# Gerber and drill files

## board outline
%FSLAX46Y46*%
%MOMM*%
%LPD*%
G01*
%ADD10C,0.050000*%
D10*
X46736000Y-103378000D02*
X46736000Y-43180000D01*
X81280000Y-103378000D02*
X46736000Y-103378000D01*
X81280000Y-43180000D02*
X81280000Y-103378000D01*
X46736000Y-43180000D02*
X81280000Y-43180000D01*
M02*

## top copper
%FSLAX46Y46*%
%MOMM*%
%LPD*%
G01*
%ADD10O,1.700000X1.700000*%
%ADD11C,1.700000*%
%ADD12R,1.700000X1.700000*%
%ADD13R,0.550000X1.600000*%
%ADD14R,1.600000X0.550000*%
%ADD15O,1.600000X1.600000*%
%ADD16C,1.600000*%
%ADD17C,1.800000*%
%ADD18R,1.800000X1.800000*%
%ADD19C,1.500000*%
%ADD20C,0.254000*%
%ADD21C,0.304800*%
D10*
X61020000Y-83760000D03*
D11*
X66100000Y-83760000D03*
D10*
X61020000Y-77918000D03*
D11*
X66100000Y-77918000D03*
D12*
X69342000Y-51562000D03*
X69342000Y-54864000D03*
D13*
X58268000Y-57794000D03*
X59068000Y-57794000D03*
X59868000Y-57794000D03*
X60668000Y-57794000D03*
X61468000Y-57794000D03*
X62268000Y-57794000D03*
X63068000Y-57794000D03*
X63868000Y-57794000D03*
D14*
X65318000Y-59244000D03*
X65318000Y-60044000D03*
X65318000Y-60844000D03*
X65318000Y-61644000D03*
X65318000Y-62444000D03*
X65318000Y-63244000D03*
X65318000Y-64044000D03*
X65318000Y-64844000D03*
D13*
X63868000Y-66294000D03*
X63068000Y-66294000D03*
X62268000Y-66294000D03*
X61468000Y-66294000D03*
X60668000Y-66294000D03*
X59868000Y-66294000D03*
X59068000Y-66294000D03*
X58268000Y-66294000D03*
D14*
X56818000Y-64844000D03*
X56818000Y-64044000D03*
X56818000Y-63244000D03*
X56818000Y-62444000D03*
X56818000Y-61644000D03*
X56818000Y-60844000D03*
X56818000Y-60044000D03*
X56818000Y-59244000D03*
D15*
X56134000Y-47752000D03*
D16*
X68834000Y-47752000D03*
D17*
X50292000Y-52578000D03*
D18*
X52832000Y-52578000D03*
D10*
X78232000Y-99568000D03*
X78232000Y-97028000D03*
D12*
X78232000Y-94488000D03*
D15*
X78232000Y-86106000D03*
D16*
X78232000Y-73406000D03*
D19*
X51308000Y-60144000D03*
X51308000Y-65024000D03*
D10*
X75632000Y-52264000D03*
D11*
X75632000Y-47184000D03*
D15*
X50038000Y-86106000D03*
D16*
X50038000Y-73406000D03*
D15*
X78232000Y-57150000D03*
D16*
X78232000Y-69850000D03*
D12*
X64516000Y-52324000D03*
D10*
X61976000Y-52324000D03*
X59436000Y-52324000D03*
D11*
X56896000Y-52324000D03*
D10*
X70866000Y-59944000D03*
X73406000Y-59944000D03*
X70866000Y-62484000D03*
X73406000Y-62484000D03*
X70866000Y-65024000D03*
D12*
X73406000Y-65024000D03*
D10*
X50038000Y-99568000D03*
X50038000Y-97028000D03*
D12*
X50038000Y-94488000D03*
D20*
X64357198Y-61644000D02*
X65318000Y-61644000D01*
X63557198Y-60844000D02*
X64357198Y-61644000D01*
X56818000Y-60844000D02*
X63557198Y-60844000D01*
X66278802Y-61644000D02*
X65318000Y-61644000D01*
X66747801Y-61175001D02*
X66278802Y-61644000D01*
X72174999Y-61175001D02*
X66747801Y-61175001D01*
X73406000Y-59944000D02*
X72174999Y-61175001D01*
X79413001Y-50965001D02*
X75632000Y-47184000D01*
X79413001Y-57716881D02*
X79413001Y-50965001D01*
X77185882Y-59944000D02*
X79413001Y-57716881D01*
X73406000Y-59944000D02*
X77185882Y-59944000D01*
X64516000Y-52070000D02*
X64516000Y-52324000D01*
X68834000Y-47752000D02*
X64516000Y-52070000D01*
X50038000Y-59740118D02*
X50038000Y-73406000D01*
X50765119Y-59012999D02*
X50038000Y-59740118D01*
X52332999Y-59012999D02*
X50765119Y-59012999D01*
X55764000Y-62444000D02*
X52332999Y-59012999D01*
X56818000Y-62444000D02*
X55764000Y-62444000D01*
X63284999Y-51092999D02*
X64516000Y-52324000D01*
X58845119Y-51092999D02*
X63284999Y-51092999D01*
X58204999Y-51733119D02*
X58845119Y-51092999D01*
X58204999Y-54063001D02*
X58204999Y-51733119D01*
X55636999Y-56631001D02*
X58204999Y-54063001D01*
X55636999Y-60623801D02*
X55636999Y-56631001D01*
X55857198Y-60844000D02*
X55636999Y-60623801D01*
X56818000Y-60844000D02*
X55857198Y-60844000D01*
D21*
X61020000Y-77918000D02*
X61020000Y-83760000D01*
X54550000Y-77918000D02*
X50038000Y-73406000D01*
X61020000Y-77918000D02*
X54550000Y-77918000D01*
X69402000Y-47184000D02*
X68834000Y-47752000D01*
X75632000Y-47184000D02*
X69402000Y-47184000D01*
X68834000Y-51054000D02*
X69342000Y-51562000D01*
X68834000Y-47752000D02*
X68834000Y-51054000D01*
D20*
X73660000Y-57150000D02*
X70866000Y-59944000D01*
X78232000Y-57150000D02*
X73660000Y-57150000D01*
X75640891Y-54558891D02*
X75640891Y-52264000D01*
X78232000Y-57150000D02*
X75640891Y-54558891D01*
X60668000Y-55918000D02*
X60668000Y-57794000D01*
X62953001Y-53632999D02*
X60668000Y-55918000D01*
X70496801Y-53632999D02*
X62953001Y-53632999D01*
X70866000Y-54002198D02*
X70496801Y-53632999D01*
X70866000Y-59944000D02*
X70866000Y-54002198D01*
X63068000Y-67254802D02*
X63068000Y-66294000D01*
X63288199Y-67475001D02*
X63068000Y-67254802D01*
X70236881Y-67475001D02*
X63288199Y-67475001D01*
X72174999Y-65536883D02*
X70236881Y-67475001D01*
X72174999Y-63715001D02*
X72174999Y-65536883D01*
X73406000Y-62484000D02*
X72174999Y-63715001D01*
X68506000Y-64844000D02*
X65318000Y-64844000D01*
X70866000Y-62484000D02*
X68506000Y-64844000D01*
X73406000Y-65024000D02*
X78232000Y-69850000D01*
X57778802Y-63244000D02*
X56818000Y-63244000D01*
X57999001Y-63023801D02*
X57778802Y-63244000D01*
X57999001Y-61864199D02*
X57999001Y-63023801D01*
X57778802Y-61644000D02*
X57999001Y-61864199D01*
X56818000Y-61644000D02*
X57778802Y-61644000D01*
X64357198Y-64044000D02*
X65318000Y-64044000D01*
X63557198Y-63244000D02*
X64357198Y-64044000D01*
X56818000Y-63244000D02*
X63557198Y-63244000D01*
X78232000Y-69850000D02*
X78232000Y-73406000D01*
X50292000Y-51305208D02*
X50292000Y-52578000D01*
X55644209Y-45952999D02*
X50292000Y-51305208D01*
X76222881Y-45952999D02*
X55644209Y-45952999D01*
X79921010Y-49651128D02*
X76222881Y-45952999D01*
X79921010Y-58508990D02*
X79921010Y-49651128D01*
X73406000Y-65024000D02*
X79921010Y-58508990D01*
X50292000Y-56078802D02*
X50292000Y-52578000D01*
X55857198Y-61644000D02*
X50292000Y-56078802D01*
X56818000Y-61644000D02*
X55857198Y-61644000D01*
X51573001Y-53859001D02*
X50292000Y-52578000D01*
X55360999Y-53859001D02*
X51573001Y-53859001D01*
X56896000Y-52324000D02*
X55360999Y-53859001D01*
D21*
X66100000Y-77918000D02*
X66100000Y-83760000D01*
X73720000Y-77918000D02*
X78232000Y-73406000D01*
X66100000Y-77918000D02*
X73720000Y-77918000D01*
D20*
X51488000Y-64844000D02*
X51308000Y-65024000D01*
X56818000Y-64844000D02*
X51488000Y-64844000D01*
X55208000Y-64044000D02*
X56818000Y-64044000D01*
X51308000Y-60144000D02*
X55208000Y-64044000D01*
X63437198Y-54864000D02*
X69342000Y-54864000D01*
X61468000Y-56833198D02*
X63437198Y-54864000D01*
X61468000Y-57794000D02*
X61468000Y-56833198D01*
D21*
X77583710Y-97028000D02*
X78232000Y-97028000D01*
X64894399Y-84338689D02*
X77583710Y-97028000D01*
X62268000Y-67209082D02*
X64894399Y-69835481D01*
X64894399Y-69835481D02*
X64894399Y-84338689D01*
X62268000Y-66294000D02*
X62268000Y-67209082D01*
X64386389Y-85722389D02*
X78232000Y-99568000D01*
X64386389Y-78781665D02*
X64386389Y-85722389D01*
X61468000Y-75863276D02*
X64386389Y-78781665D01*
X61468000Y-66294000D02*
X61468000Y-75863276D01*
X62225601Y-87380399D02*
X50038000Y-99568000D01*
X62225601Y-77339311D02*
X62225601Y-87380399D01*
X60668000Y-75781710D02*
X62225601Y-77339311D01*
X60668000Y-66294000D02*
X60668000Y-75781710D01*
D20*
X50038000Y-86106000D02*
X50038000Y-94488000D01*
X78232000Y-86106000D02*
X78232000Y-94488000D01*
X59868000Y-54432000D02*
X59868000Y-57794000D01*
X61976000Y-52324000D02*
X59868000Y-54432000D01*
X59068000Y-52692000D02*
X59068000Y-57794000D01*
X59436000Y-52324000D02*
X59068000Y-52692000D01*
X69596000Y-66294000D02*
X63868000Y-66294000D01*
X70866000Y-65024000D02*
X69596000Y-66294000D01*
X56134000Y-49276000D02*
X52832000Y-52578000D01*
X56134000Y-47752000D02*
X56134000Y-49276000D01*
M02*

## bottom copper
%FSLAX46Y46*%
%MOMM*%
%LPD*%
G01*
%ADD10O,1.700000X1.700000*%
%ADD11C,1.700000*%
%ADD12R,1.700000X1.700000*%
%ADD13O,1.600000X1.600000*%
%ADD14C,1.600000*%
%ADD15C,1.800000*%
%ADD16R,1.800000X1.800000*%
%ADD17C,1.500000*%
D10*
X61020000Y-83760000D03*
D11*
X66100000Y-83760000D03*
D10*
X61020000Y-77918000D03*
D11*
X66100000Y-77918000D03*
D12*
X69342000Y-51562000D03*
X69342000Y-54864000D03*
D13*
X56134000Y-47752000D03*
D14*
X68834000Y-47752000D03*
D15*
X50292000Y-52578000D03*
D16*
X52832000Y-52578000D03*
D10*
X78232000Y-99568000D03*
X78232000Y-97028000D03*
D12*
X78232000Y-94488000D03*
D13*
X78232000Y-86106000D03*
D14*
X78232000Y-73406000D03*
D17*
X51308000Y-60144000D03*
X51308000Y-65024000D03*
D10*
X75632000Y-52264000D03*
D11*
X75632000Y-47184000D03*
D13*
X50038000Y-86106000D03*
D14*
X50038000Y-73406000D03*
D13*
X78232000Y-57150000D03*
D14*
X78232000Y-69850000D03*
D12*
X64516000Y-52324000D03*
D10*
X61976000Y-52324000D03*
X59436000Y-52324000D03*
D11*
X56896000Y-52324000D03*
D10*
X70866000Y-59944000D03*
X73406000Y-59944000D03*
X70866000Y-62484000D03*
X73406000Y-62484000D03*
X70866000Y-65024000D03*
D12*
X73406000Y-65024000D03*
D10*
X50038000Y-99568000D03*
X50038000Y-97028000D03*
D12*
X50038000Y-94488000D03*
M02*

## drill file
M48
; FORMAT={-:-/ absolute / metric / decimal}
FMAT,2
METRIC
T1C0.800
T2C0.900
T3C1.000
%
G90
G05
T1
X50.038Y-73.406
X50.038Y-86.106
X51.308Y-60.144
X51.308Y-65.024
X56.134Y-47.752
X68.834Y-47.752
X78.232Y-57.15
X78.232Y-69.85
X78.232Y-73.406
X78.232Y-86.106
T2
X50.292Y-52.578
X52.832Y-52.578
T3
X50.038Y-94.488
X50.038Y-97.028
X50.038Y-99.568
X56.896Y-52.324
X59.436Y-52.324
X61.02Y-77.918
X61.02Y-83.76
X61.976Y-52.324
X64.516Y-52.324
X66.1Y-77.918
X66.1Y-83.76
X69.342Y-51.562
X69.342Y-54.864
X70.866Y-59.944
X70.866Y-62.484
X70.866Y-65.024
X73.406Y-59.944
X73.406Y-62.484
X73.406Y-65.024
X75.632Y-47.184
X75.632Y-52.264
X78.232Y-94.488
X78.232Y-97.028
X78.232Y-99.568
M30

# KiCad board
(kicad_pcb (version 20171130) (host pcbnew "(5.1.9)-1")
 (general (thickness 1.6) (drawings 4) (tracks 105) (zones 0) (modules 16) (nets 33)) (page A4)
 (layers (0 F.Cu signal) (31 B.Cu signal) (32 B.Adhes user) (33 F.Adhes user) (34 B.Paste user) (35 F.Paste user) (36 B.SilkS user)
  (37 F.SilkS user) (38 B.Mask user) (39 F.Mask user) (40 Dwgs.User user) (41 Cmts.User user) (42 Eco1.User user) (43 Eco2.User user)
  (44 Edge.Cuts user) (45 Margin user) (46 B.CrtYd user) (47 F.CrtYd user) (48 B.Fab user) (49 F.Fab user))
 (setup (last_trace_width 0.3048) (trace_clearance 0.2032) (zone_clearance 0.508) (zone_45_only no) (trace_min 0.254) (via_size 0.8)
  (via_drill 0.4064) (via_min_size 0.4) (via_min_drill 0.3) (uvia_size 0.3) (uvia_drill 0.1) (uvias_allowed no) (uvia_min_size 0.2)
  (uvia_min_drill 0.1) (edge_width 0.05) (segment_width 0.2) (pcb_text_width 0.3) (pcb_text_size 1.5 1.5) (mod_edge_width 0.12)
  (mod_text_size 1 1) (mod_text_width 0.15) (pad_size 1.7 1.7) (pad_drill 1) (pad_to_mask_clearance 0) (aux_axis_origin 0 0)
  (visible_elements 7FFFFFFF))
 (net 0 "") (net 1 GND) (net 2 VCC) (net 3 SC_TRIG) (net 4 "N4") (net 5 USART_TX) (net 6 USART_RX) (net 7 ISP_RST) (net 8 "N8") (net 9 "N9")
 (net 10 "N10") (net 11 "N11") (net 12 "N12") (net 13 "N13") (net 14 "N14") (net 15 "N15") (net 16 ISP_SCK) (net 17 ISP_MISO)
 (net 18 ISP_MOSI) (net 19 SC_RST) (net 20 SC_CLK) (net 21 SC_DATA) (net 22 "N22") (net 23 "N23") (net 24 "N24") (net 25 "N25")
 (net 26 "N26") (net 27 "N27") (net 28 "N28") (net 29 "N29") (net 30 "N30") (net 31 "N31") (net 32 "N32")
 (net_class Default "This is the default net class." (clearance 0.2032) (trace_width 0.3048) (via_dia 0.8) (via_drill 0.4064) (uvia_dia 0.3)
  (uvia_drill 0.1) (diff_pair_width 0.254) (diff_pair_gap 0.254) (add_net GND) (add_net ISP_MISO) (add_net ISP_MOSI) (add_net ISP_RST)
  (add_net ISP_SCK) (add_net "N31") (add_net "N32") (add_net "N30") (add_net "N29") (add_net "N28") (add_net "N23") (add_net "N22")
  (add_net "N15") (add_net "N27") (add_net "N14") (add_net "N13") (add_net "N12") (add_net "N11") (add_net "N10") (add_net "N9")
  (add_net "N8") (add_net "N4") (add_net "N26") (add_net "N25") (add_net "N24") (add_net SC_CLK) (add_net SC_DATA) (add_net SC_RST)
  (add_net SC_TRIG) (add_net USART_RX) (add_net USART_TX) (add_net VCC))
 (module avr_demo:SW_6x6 (layer F.Cu) (at 66.04 81.28 270)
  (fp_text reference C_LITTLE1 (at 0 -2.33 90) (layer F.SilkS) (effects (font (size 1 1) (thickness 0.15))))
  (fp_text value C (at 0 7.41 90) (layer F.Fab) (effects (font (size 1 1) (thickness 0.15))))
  (pad 2 thru_hole oval (at 2.48 5.02 270) (size 1.7 1.7) (drill 1) (layers *.Cu *.Mask) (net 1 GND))
  (pad 1 thru_hole circle (at 2.48 -0.06 270) (size 1.7 1.7) (drill 1) (layers *.Cu *.Mask) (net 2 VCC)))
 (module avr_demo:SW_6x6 (layer F.Cu) (at 66.04 75.438 270)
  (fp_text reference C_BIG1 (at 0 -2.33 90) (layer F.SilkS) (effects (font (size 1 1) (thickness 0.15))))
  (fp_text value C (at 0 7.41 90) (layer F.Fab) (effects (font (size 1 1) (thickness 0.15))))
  (pad 2 thru_hole oval (at 2.48 5.02 270) (size 1.7 1.7) (drill 1) (layers *.Cu *.Mask) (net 1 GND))
  (pad 1 thru_hole circle (at 2.48 -0.06 270) (size 1.7 1.7) (drill 1) (layers *.Cu *.Mask) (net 2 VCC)))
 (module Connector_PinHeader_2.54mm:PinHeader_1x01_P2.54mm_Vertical (layer F.Cu) (at 69.342 51.562)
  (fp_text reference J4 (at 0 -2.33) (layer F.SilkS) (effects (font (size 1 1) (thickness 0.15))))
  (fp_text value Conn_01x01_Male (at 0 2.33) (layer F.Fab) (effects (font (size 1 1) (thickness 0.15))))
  (pad 1 thru_hole rect (at 0 0) (size 1.7 1.7) (drill 1) (layers *.Cu *.Mask) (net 1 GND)))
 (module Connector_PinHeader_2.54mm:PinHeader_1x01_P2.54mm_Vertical (layer F.Cu) (at 69.342 54.864)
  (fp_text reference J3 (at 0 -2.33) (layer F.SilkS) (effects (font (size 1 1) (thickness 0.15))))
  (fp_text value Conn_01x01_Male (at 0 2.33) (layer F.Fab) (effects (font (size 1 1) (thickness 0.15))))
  (pad 1 thru_hole rect (at 0 0) (size 1.7 1.7) (drill 1) (layers *.Cu *.Mask) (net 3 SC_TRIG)))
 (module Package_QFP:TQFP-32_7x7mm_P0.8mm (layer F.Cu) (at 61.068 62.044)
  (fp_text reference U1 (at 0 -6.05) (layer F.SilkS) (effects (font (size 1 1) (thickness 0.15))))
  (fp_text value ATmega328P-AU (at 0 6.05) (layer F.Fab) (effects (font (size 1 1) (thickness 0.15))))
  (pad 32 smd rect (at -2.8 -4.25 90) (size 1.6 0.55) (layers F.Cu F.Paste F.Mask) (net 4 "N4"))
  (pad 31 smd rect (at -2 -4.25 90) (size 1.6 0.55) (layers F.Cu F.Paste F.Mask) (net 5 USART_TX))
  (pad 30 smd rect (at -1.2 -4.25 90) (size 1.6 0.55) (layers F.Cu F.Paste F.Mask) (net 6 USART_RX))
  (pad 29 smd rect (at -0.4 -4.25 90) (size 1.6 0.55) (layers F.Cu F.Paste F.Mask) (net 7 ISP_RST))
  (pad 28 smd rect (at 0.4 -4.25 90) (size 1.6 0.55) (layers F.Cu F.Paste F.Mask) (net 3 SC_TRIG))
  (pad 27 smd rect (at 1.2 -4.25 90) (size 1.6 0.55) (layers F.Cu F.Paste F.Mask) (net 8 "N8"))
  (pad 26 smd rect (at 2 -4.25 90) (size 1.6 0.55) (layers F.Cu F.Paste F.Mask) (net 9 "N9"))
  (pad 25 smd rect (at 2.8 -4.25 90) (size 1.6 0.55) (layers F.Cu F.Paste F.Mask) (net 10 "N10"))
  (pad 24 smd rect (at 4.25 -2.8) (size 1.6 0.55) (layers F.Cu F.Paste F.Mask) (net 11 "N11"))
  (pad 23 smd rect (at 4.25 -2) (size 1.6 0.55) (layers F.Cu F.Paste F.Mask) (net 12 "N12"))
  (pad 22 smd rect (at 4.25 -1.2) (size 1.6 0.55) (layers F.Cu F.Paste F.Mask) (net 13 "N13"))
  (pad 21 smd rect (at 4.25 -0.4) (size 1.6 0.55) (layers F.Cu F.Paste F.Mask) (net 1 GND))
  (pad 20 smd rect (at 4.25 0.4) (size 1.6 0.55) (layers F.Cu F.Paste F.Mask) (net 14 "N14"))
  (pad 19 smd rect (at 4.25 1.2) (size 1.6 0.55) (layers F.Cu F.Paste F.Mask) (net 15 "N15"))
  (pad 18 smd rect (at 4.25 2) (size 1.6 0.55) (layers F.Cu F.Paste F.Mask) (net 2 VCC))
  (pad 17 smd rect (at 4.25 2.8) (size 1.6 0.55) (layers F.Cu F.Paste F.Mask) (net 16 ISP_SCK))
  (pad 16 smd rect (at 2.8 4.25 90) (size 1.6 0.55) (layers F.Cu F.Paste F.Mask) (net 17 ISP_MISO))
  (pad 15 smd rect (at 2 4.25 90) (size 1.6 0.55) (layers F.Cu F.Paste F.Mask) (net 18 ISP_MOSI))
  (pad 14 smd rect (at 1.2 4.25 90) (size 1.6 0.55) (layers F.Cu F.Paste F.Mask) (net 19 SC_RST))
  (pad 13 smd rect (at 0.4 4.25 90) (size 1.6 0.55) (layers F.Cu F.Paste F.Mask) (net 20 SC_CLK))
  (pad 12 smd rect (at -0.4 4.25 90) (size 1.6 0.55) (layers F.Cu F.Paste F.Mask) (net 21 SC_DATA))
  (pad 11 smd rect (at -1.2 4.25 90) (size 1.6 0.55) (layers F.Cu F.Paste F.Mask) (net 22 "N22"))
  (pad 10 smd rect (at -2 4.25 90) (size 1.6 0.55) (layers F.Cu F.Paste F.Mask) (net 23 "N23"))
  (pad 9 smd rect (at -2.8 4.25 90) (size 1.6 0.55) (layers F.Cu F.Paste F.Mask) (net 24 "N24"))
  (pad 8 smd rect (at -4.25 2.8) (size 1.6 0.55) (layers F.Cu F.Paste F.Mask) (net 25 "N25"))
  (pad 7 smd rect (at -4.25 2) (size 1.6 0.55) (layers F.Cu F.Paste F.Mask) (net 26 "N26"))
  (pad 6 smd rect (at -4.25 1.2) (size 1.6 0.55) (layers F.Cu F.Paste F.Mask) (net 2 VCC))
  (pad 5 smd rect (at -4.25 0.4) (size 1.6 0.55) (layers F.Cu F.Paste F.Mask) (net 1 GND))
  (pad 4 smd rect (at -4.25 -0.4) (size 1.6 0.55) (layers F.Cu F.Paste F.Mask) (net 2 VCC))
  (pad 3 smd rect (at -4.25 -1.2) (size 1.6 0.55) (layers F.Cu F.Paste F.Mask) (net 1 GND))
  (pad 2 smd rect (at -4.25 -2) (size 1.6 0.55) (layers F.Cu F.Paste F.Mask) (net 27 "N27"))
  (pad 1 smd rect (at -4.25 -2.8) (size 1.6 0.55) (layers F.Cu F.Paste F.Mask) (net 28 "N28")))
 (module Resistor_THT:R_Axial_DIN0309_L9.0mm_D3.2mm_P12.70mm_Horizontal (layer F.Cu) (at 68.834 47.752 180)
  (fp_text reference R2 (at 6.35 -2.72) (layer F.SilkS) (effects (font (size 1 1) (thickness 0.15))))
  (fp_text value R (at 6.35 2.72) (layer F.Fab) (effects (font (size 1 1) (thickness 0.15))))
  (pad 2 thru_hole oval (at 12.7 0 180) (size 1.6 1.6) (drill 0.8) (layers *.Cu *.Mask) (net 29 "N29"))
  (pad 1 thru_hole circle (at 0 0 180) (size 1.6 1.6) (drill 0.8) (layers *.Cu *.Mask) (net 1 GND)))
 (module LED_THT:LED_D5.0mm (layer F.Cu) (at 52.832 52.578 180)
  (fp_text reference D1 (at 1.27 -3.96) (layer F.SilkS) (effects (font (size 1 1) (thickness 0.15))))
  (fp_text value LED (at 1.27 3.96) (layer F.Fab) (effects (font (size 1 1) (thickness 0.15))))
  (pad 2 thru_hole circle (at 2.54 0 180) (size 1.8 1.8) (drill 0.9) (layers *.Cu *.Mask) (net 2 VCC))
  (pad 1 thru_hole rect (at 0 0 180) (size 1.8 1.8) (drill 0.9) (layers *.Cu *.Mask) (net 29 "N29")))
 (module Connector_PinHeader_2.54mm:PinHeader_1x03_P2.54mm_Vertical (layer F.Cu) (at 78.232 94.488)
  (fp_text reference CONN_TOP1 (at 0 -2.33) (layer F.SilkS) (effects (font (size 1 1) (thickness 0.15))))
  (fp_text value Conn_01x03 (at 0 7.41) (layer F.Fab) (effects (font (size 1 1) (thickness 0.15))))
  (pad 3 thru_hole oval (at 0 5.08) (size 1.7 1.7) (drill 1) (layers *.Cu *.Mask) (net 20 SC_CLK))
  (pad 2 thru_hole oval (at 0 2.54) (size 1.7 1.7) (drill 1) (layers *.Cu *.Mask) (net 19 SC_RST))
  (pad 1 thru_hole rect (at 0 0) (size 1.7 1.7) (drill 1) (layers *.Cu *.Mask) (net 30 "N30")))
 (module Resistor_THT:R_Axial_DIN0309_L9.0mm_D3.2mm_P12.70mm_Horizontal (layer F.Cu) (at 78.232 73.406 270)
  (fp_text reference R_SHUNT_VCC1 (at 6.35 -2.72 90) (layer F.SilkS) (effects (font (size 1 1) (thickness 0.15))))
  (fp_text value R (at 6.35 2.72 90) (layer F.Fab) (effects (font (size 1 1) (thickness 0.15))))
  (pad 2 thru_hole oval (at 12.7 0 270) (size 1.6 1.6) (drill 0.8) (layers *.Cu *.Mask) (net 30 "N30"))
  (pad 1 thru_hole circle (at 0 0 270) (size 1.6 1.6) (drill 0.8) (layers *.Cu *.Mask) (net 2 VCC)))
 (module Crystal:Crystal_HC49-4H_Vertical (layer F.Cu) (at 51.308 65.024 90)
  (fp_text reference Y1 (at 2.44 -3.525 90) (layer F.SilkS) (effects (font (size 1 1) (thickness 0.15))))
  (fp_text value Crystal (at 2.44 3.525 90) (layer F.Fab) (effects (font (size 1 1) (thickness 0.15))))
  (pad 2 thru_hole circle (at 4.88 0 90) (size 1.5 1.5) (drill 0.8) (layers *.Cu *.Mask) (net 26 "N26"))
  (pad 1 thru_hole circle (at 0 0 90) (size 1.5 1.5) (drill 0.8) (layers *.Cu *.Mask) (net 25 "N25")))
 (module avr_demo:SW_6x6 (layer F.Cu) (at 73.152 47.244)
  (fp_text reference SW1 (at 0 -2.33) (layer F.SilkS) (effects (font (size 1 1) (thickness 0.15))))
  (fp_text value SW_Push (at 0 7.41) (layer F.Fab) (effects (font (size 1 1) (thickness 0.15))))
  (pad 2 thru_hole oval (at 2.48 5.02) (size 1.7 1.7) (drill 1) (layers *.Cu *.Mask) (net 7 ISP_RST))
  (pad 1 thru_hole circle (at 2.48 -0.06) (size 1.7 1.7) (drill 1) (layers *.Cu *.Mask) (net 1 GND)))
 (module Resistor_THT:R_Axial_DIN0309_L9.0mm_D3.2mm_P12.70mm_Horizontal (layer F.Cu) (at 50.038 73.406 270)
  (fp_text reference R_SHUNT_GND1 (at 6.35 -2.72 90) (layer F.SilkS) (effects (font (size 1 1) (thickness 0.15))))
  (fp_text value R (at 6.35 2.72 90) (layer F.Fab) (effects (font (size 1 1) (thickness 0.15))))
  (pad 2 thru_hole oval (at 12.7 0 270) (size 1.6 1.6) (drill 0.8) (layers *.Cu *.Mask) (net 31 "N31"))
  (pad 1 thru_hole circle (at 0 0 270) (size 1.6 1.6) (drill 0.8) (layers *.Cu *.Mask) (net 1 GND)))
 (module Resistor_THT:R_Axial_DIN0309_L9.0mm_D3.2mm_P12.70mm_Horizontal (layer F.Cu) (at 78.232 69.85 90)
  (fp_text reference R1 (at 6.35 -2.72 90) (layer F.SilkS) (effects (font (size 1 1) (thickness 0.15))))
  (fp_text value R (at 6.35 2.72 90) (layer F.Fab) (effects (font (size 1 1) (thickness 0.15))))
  (pad 2 thru_hole oval (at 12.7 0 90) (size 1.6 1.6) (drill 0.8) (layers *.Cu *.Mask) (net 7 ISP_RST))
  (pad 1 thru_hole circle (at 0 0 90) (size 1.6 1.6) (drill 0.8) (layers *.Cu *.Mask) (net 2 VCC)))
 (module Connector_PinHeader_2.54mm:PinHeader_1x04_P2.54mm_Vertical (layer F.Cu) (at 56.896 52.324 90)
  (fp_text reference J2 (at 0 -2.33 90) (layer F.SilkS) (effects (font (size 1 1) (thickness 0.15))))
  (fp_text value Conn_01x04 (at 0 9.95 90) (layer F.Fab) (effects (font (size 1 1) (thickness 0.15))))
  (pad 4 thru_hole rect (at 0 7.62 90) (size 1.7 1.7) (drill 1) (layers *.Cu *.Mask) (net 1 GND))
  (pad 3 thru_hole oval (at 0 5.08 90) (size 1.7 1.7) (drill 1) (layers *.Cu *.Mask) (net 6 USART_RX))
  (pad 2 thru_hole oval (at 0 2.54 90) (size 1.7 1.7) (drill 1) (layers *.Cu *.Mask) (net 5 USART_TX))
  (pad 1 thru_hole circle (at 0 0 90) (size 1.7 1.7) (drill 1) (layers *.Cu *.Mask) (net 2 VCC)))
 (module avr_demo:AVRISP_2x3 (layer F.Cu) (at 73.406 65.024 180)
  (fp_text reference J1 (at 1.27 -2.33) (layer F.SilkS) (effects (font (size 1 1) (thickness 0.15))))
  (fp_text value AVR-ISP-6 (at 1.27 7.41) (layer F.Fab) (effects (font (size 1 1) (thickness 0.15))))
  (pad 5 thru_hole oval (at 2.54 5.08 180) (size 1.7 1.7) (drill 1) (layers *.Cu *.Mask) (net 7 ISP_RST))
  (pad 6 thru_hole oval (at 0 5.08 180) (size 1.7 1.7) (drill 1) (layers *.Cu *.Mask) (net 1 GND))
  (pad 3 thru_hole oval (at 2.54 2.54 180) (size 1.7 1.7) (drill 1) (layers *.Cu *.Mask) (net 16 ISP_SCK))
  (pad 4 thru_hole oval (at 0 2.54 180) (size 1.7 1.7) (drill 1) (layers *.Cu *.Mask) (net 18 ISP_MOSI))
  (pad 1 thru_hole oval (at 2.54 0 180) (size 1.7 1.7) (drill 1) (layers *.Cu *.Mask) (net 17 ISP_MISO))
  (pad 2 thru_hole rect (at 0 0 180) (size 1.7 1.7) (drill 1) (layers *.Cu *.Mask) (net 2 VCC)))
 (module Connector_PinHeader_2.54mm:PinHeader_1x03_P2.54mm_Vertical (layer F.Cu) (at 50.038 94.488)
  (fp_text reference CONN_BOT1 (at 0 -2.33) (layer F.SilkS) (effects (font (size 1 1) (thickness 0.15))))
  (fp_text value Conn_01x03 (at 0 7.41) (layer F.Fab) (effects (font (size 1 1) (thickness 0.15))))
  (pad 3 thru_hole oval (at 0 5.08) (size 1.7 1.7) (drill 1) (layers *.Cu *.Mask) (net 21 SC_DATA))
  (pad 2 thru_hole oval (at 0 2.54) (size 1.7 1.7) (drill 1) (layers *.Cu *.Mask) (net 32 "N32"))
  (pad 1 thru_hole rect (at 0 0) (size 1.7 1.7) (drill 1) (layers *.Cu *.Mask) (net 31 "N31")))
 (gr_line (start 46.736 103.378) (end 46.736 43.18) (layer Edge.Cuts) (width 0.05))
 (gr_line (start 81.28 103.378) (end 46.736 103.378) (layer Edge.Cuts) (width 0.05))
 (gr_line (start 81.28 43.18) (end 81.28 103.378) (layer Edge.Cuts) (width 0.05))
 (gr_line (start 46.736 43.18) (end 81.28 43.18) (layer Edge.Cuts) (width 0.05))
 (segment (start 64.357198 61.644) (end 65.318 61.644) (width 0.254) (layer F.Cu) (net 1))
 (segment (start 63.557198 60.844) (end 64.357198 61.644) (width 0.254) (layer F.Cu) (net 1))
 (segment (start 56.818 60.844) (end 63.557198 60.844) (width 0.254) (layer F.Cu) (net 1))
 (segment (start 66.278802 61.644) (end 65.318 61.644) (width 0.254) (layer F.Cu) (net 1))
 (segment (start 66.747801 61.175001) (end 66.278802 61.644) (width 0.254) (layer F.Cu) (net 1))
 (segment (start 72.174999 61.175001) (end 66.747801 61.175001) (width 0.254) (layer F.Cu) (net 1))
 (segment (start 73.406 59.944) (end 72.174999 61.175001) (width 0.254) (layer F.Cu) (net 1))
 (segment (start 79.413001 50.965001) (end 75.632 47.184) (width 0.254) (layer F.Cu) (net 1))
 (segment (start 79.413001 57.716881) (end 79.413001 50.965001) (width 0.254) (layer F.Cu) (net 1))
 (segment (start 77.185882 59.944) (end 79.413001 57.716881) (width 0.254) (layer F.Cu) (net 1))
 (segment (start 73.406 59.944) (end 77.185882 59.944) (width 0.254) (layer F.Cu) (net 1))
 (segment (start 64.516 52.07) (end 64.516 52.324) (width 0.254) (layer F.Cu) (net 1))
 (segment (start 68.834 47.752) (end 64.516 52.07) (width 0.254) (layer F.Cu) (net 1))
 (segment (start 50.038 59.740118) (end 50.038 73.406) (width 0.254) (layer F.Cu) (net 1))
 (segment (start 50.765119 59.012999) (end 50.038 59.740118) (width 0.254) (layer F.Cu) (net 1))
 (segment (start 52.332999 59.012999) (end 50.765119 59.012999) (width 0.254) (layer F.Cu) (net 1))
 (segment (start 55.764 62.444) (end 52.332999 59.012999) (width 0.254) (layer F.Cu) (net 1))
 (segment (start 56.818 62.444) (end 55.764 62.444) (width 0.254) (layer F.Cu) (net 1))
 (segment (start 63.284999 51.092999) (end 64.516 52.324) (width 0.254) (layer F.Cu) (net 1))
 (segment (start 58.845119 51.092999) (end 63.284999 51.092999) (width 0.254) (layer F.Cu) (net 1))
 (segment (start 58.204999 51.733119) (end 58.845119 51.092999) (width 0.254) (layer F.Cu) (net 1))
 (segment (start 58.204999 54.063001) (end 58.204999 51.733119) (width 0.254) (layer F.Cu) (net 1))
 (segment (start 55.636999 56.631001) (end 58.204999 54.063001) (width 0.254) (layer F.Cu) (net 1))
 (segment (start 55.636999 60.623801) (end 55.636999 56.631001) (width 0.254) (layer F.Cu) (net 1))
 (segment (start 55.857198 60.844) (end 55.636999 60.623801) (width 0.254) (layer F.Cu) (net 1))
 (segment (start 56.818 60.844) (end 55.857198 60.844) (width 0.254) (layer F.Cu) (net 1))
 (segment (start 61.02 77.918) (end 61.02 83.76) (width 0.3048) (layer F.Cu) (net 1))
 (segment (start 54.55 77.918) (end 50.038 73.406) (width 0.3048) (layer F.Cu) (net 1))
 (segment (start 61.02 77.918) (end 54.55 77.918) (width 0.3048) (layer F.Cu) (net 1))
 (segment (start 69.402 47.184) (end 68.834 47.752) (width 0.3048) (layer F.Cu) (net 1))
 (segment (start 75.632 47.184) (end 69.402 47.184) (width 0.3048) (layer F.Cu) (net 1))
 (segment (start 68.834 51.054) (end 69.342 51.562) (width 0.3048) (layer F.Cu) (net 1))
 (segment (start 68.834 47.752) (end 68.834 51.054) (width 0.3048) (layer F.Cu) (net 1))
 (segment (start 73.66 57.15) (end 70.866 59.944) (width 0.254) (layer F.Cu) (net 7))
 (segment (start 78.232 57.15) (end 73.66 57.15) (width 0.254) (layer F.Cu) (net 7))
 (segment (start 75.640891 54.558891) (end 75.640891 52.264) (width 0.254) (layer F.Cu) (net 7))
 (segment (start 78.232 57.15) (end 75.640891 54.558891) (width 0.254) (layer F.Cu) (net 7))
 (segment (start 60.668 55.918) (end 60.668 57.794) (width 0.254) (layer F.Cu) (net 7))
 (segment (start 62.953001 53.632999) (end 60.668 55.918) (width 0.254) (layer F.Cu) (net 7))
 (segment (start 70.496801 53.632999) (end 62.953001 53.632999) (width 0.254) (layer F.Cu) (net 7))
 (segment (start 70.866 54.002198) (end 70.496801 53.632999) (width 0.254) (layer F.Cu) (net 7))
 (segment (start 70.866 59.944) (end 70.866 54.002198) (width 0.254) (layer F.Cu) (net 7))
 (segment (start 63.068 67.254802) (end 63.068 66.294) (width 0.254) (layer F.Cu) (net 18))
 (segment (start 63.288199 67.475001) (end 63.068 67.254802) (width 0.254) (layer F.Cu) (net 18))
 (segment (start 70.236881 67.475001) (end 63.288199 67.475001) (width 0.254) (layer F.Cu) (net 18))
 (segment (start 72.174999 65.536883) (end 70.236881 67.475001) (width 0.254) (layer F.Cu) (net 18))
 (segment (start 72.174999 63.715001) (end 72.174999 65.536883) (width 0.254) (layer F.Cu) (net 18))
 (segment (start 73.406 62.484) (end 72.174999 63.715001) (width 0.254) (layer F.Cu) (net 18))
 (segment (start 68.506 64.844) (end 65.318 64.844) (width 0.254) (layer F.Cu) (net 16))
 (segment (start 70.866 62.484) (end 68.506 64.844) (width 0.254) (layer F.Cu) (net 16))
 (segment (start 73.406 65.024) (end 78.232 69.85) (width 0.254) (layer F.Cu) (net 2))
 (segment (start 57.778802 63.244) (end 56.818 63.244) (width 0.254) (layer F.Cu) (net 2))
 (segment (start 57.999001 63.023801) (end 57.778802 63.244) (width 0.254) (layer F.Cu) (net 2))
 (segment (start 57.999001 61.864199) (end 57.999001 63.023801) (width 0.254) (layer F.Cu) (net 2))
 (segment (start 57.778802 61.644) (end 57.999001 61.864199) (width 0.254) (layer F.Cu) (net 2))
 (segment (start 56.818 61.644) (end 57.778802 61.644) (width 0.254) (layer F.Cu) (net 2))
 (segment (start 64.357198 64.044) (end 65.318 64.044) (width 0.254) (layer F.Cu) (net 2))
 (segment (start 63.557198 63.244) (end 64.357198 64.044) (width 0.254) (layer F.Cu) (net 2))
 (segment (start 56.818 63.244) (end 63.557198 63.244) (width 0.254) (layer F.Cu) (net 2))
 (segment (start 78.232 69.85) (end 78.232 73.406) (width 0.254) (layer F.Cu) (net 2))
 (segment (start 50.292 51.305208) (end 50.292 52.578) (width 0.254) (layer F.Cu) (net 2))
 (segment (start 55.644209 45.952999) (end 50.292 51.305208) (width 0.254) (layer F.Cu) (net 2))
 (segment (start 76.222881 45.952999) (end 55.644209 45.952999) (width 0.254) (layer F.Cu) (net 2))
 (segment (start 79.92101 49.651128) (end 76.222881 45.952999) (width 0.254) (layer F.Cu) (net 2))
 (segment (start 79.92101 58.50899) (end 79.92101 49.651128) (width 0.254) (layer F.Cu) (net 2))
 (segment (start 73.406 65.024) (end 79.92101 58.50899) (width 0.254) (layer F.Cu) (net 2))
 (segment (start 50.292 56.078802) (end 50.292 52.578) (width 0.254) (layer F.Cu) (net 2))
 (segment (start 55.857198 61.644) (end 50.292 56.078802) (width 0.254) (layer F.Cu) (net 2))
 (segment (start 56.818 61.644) (end 55.857198 61.644) (width 0.254) (layer F.Cu) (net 2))
 (segment (start 51.573001 53.859001) (end 50.292 52.578) (width 0.254) (layer F.Cu) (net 2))
 (segment (start 55.360999 53.859001) (end 51.573001 53.859001) (width 0.254) (layer F.Cu) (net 2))
 (segment (start 56.896 52.324) (end 55.360999 53.859001) (width 0.254) (layer F.Cu) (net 2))
 (segment (start 66.1 77.918) (end 66.1 83.76) (width 0.3048) (layer F.Cu) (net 2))
 (segment (start 73.72 77.918) (end 78.232 73.406) (width 0.3048) (layer F.Cu) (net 2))
 (segment (start 66.1 77.918) (end 73.72 77.918) (width 0.3048) (layer F.Cu) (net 2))
 (segment (start 51.488 64.844) (end 51.308 65.024) (width 0.254) (layer F.Cu) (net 25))
 (segment (start 56.818 64.844) (end 51.488 64.844) (width 0.254) (layer F.Cu) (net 25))
 (segment (start 55.208 64.044) (end 56.818 64.044) (width 0.254) (layer F.Cu) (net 26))
 (segment (start 51.308 60.144) (end 55.208 64.044) (width 0.254) (layer F.Cu) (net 26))
 (segment (start 63.437198 54.864) (end 69.342 54.864) (width 0.254) (layer F.Cu) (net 3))
 (segment (start 61.468 56.833198) (end 63.437198 54.864) (width 0.254) (layer F.Cu) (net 3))
 (segment (start 61.468 57.794) (end 61.468 56.833198) (width 0.254) (layer F.Cu) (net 3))
 (segment (start 77.58371 97.028) (end 78.232 97.028) (width 0.3048) (layer F.Cu) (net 19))
 (segment (start 64.894399 84.338689) (end 77.58371 97.028) (width 0.3048) (layer F.Cu) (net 19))
 (segment (start 62.268 67.209082) (end 64.894399 69.835481) (width 0.3048) (layer F.Cu) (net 19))
 (segment (start 64.894399 69.835481) (end 64.894399 84.338689) (width 0.3048) (layer F.Cu) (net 19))
 (segment (start 62.268 66.294) (end 62.268 67.209082) (width 0.3048) (layer F.Cu) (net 19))
 (segment (start 64.386389 85.722389) (end 78.232 99.568) (width 0.3048) (layer F.Cu) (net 20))
 (segment (start 64.386389 78.781665) (end 64.386389 85.722389) (width 0.3048) (layer F.Cu) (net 20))
 (segment (start 61.468 75.863276) (end 64.386389 78.781665) (width 0.3048) (layer F.Cu) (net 20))
 (segment (start 61.468 66.294) (end 61.468 75.863276) (width 0.3048) (layer F.Cu) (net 20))
 (segment (start 62.225601 87.380399) (end 50.038 99.568) (width 0.3048) (layer F.Cu) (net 21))
 (segment (start 62.225601 77.339311) (end 62.225601 87.380399) (width 0.3048) (layer F.Cu) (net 21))
 (segment (start 60.668 75.78171) (end 62.225601 77.339311) (width 0.3048) (layer F.Cu) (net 21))
 (segment (start 60.668 66.294) (end 60.668 75.78171) (width 0.3048) (layer F.Cu) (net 21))
 (segment (start 50.038 86.106) (end 50.038 94.488) (width 0.254) (layer F.Cu) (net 31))
 (segment (start 78.232 86.106) (end 78.232 94.488) (width 0.254) (layer F.Cu) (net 30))
 (segment (start 59.868 54.432) (end 59.868 57.794) (width 0.254) (layer F.Cu) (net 6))
 (segment (start 61.976 52.324) (end 59.868 54.432) (width 0.254) (layer F.Cu) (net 6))
 (segment (start 59.068 52.692) (end 59.068 57.794) (width 0.254) (layer F.Cu) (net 5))
 (segment (start 59.436 52.324) (end 59.068 52.692) (width 0.254) (layer F.Cu) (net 5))
 (segment (start 69.596 66.294) (end 63.868 66.294) (width 0.254) (layer F.Cu) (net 17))
 (segment (start 70.866 65.024) (end 69.596 66.294) (width 0.254) (layer F.Cu) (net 17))
 (segment (start 56.134 49.276) (end 52.832 52.578) (width 0.254) (layer F.Cu) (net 29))
 (segment (start 56.134 47.752) (end 56.134 49.276) (width 0.254) (layer F.Cu) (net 29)))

